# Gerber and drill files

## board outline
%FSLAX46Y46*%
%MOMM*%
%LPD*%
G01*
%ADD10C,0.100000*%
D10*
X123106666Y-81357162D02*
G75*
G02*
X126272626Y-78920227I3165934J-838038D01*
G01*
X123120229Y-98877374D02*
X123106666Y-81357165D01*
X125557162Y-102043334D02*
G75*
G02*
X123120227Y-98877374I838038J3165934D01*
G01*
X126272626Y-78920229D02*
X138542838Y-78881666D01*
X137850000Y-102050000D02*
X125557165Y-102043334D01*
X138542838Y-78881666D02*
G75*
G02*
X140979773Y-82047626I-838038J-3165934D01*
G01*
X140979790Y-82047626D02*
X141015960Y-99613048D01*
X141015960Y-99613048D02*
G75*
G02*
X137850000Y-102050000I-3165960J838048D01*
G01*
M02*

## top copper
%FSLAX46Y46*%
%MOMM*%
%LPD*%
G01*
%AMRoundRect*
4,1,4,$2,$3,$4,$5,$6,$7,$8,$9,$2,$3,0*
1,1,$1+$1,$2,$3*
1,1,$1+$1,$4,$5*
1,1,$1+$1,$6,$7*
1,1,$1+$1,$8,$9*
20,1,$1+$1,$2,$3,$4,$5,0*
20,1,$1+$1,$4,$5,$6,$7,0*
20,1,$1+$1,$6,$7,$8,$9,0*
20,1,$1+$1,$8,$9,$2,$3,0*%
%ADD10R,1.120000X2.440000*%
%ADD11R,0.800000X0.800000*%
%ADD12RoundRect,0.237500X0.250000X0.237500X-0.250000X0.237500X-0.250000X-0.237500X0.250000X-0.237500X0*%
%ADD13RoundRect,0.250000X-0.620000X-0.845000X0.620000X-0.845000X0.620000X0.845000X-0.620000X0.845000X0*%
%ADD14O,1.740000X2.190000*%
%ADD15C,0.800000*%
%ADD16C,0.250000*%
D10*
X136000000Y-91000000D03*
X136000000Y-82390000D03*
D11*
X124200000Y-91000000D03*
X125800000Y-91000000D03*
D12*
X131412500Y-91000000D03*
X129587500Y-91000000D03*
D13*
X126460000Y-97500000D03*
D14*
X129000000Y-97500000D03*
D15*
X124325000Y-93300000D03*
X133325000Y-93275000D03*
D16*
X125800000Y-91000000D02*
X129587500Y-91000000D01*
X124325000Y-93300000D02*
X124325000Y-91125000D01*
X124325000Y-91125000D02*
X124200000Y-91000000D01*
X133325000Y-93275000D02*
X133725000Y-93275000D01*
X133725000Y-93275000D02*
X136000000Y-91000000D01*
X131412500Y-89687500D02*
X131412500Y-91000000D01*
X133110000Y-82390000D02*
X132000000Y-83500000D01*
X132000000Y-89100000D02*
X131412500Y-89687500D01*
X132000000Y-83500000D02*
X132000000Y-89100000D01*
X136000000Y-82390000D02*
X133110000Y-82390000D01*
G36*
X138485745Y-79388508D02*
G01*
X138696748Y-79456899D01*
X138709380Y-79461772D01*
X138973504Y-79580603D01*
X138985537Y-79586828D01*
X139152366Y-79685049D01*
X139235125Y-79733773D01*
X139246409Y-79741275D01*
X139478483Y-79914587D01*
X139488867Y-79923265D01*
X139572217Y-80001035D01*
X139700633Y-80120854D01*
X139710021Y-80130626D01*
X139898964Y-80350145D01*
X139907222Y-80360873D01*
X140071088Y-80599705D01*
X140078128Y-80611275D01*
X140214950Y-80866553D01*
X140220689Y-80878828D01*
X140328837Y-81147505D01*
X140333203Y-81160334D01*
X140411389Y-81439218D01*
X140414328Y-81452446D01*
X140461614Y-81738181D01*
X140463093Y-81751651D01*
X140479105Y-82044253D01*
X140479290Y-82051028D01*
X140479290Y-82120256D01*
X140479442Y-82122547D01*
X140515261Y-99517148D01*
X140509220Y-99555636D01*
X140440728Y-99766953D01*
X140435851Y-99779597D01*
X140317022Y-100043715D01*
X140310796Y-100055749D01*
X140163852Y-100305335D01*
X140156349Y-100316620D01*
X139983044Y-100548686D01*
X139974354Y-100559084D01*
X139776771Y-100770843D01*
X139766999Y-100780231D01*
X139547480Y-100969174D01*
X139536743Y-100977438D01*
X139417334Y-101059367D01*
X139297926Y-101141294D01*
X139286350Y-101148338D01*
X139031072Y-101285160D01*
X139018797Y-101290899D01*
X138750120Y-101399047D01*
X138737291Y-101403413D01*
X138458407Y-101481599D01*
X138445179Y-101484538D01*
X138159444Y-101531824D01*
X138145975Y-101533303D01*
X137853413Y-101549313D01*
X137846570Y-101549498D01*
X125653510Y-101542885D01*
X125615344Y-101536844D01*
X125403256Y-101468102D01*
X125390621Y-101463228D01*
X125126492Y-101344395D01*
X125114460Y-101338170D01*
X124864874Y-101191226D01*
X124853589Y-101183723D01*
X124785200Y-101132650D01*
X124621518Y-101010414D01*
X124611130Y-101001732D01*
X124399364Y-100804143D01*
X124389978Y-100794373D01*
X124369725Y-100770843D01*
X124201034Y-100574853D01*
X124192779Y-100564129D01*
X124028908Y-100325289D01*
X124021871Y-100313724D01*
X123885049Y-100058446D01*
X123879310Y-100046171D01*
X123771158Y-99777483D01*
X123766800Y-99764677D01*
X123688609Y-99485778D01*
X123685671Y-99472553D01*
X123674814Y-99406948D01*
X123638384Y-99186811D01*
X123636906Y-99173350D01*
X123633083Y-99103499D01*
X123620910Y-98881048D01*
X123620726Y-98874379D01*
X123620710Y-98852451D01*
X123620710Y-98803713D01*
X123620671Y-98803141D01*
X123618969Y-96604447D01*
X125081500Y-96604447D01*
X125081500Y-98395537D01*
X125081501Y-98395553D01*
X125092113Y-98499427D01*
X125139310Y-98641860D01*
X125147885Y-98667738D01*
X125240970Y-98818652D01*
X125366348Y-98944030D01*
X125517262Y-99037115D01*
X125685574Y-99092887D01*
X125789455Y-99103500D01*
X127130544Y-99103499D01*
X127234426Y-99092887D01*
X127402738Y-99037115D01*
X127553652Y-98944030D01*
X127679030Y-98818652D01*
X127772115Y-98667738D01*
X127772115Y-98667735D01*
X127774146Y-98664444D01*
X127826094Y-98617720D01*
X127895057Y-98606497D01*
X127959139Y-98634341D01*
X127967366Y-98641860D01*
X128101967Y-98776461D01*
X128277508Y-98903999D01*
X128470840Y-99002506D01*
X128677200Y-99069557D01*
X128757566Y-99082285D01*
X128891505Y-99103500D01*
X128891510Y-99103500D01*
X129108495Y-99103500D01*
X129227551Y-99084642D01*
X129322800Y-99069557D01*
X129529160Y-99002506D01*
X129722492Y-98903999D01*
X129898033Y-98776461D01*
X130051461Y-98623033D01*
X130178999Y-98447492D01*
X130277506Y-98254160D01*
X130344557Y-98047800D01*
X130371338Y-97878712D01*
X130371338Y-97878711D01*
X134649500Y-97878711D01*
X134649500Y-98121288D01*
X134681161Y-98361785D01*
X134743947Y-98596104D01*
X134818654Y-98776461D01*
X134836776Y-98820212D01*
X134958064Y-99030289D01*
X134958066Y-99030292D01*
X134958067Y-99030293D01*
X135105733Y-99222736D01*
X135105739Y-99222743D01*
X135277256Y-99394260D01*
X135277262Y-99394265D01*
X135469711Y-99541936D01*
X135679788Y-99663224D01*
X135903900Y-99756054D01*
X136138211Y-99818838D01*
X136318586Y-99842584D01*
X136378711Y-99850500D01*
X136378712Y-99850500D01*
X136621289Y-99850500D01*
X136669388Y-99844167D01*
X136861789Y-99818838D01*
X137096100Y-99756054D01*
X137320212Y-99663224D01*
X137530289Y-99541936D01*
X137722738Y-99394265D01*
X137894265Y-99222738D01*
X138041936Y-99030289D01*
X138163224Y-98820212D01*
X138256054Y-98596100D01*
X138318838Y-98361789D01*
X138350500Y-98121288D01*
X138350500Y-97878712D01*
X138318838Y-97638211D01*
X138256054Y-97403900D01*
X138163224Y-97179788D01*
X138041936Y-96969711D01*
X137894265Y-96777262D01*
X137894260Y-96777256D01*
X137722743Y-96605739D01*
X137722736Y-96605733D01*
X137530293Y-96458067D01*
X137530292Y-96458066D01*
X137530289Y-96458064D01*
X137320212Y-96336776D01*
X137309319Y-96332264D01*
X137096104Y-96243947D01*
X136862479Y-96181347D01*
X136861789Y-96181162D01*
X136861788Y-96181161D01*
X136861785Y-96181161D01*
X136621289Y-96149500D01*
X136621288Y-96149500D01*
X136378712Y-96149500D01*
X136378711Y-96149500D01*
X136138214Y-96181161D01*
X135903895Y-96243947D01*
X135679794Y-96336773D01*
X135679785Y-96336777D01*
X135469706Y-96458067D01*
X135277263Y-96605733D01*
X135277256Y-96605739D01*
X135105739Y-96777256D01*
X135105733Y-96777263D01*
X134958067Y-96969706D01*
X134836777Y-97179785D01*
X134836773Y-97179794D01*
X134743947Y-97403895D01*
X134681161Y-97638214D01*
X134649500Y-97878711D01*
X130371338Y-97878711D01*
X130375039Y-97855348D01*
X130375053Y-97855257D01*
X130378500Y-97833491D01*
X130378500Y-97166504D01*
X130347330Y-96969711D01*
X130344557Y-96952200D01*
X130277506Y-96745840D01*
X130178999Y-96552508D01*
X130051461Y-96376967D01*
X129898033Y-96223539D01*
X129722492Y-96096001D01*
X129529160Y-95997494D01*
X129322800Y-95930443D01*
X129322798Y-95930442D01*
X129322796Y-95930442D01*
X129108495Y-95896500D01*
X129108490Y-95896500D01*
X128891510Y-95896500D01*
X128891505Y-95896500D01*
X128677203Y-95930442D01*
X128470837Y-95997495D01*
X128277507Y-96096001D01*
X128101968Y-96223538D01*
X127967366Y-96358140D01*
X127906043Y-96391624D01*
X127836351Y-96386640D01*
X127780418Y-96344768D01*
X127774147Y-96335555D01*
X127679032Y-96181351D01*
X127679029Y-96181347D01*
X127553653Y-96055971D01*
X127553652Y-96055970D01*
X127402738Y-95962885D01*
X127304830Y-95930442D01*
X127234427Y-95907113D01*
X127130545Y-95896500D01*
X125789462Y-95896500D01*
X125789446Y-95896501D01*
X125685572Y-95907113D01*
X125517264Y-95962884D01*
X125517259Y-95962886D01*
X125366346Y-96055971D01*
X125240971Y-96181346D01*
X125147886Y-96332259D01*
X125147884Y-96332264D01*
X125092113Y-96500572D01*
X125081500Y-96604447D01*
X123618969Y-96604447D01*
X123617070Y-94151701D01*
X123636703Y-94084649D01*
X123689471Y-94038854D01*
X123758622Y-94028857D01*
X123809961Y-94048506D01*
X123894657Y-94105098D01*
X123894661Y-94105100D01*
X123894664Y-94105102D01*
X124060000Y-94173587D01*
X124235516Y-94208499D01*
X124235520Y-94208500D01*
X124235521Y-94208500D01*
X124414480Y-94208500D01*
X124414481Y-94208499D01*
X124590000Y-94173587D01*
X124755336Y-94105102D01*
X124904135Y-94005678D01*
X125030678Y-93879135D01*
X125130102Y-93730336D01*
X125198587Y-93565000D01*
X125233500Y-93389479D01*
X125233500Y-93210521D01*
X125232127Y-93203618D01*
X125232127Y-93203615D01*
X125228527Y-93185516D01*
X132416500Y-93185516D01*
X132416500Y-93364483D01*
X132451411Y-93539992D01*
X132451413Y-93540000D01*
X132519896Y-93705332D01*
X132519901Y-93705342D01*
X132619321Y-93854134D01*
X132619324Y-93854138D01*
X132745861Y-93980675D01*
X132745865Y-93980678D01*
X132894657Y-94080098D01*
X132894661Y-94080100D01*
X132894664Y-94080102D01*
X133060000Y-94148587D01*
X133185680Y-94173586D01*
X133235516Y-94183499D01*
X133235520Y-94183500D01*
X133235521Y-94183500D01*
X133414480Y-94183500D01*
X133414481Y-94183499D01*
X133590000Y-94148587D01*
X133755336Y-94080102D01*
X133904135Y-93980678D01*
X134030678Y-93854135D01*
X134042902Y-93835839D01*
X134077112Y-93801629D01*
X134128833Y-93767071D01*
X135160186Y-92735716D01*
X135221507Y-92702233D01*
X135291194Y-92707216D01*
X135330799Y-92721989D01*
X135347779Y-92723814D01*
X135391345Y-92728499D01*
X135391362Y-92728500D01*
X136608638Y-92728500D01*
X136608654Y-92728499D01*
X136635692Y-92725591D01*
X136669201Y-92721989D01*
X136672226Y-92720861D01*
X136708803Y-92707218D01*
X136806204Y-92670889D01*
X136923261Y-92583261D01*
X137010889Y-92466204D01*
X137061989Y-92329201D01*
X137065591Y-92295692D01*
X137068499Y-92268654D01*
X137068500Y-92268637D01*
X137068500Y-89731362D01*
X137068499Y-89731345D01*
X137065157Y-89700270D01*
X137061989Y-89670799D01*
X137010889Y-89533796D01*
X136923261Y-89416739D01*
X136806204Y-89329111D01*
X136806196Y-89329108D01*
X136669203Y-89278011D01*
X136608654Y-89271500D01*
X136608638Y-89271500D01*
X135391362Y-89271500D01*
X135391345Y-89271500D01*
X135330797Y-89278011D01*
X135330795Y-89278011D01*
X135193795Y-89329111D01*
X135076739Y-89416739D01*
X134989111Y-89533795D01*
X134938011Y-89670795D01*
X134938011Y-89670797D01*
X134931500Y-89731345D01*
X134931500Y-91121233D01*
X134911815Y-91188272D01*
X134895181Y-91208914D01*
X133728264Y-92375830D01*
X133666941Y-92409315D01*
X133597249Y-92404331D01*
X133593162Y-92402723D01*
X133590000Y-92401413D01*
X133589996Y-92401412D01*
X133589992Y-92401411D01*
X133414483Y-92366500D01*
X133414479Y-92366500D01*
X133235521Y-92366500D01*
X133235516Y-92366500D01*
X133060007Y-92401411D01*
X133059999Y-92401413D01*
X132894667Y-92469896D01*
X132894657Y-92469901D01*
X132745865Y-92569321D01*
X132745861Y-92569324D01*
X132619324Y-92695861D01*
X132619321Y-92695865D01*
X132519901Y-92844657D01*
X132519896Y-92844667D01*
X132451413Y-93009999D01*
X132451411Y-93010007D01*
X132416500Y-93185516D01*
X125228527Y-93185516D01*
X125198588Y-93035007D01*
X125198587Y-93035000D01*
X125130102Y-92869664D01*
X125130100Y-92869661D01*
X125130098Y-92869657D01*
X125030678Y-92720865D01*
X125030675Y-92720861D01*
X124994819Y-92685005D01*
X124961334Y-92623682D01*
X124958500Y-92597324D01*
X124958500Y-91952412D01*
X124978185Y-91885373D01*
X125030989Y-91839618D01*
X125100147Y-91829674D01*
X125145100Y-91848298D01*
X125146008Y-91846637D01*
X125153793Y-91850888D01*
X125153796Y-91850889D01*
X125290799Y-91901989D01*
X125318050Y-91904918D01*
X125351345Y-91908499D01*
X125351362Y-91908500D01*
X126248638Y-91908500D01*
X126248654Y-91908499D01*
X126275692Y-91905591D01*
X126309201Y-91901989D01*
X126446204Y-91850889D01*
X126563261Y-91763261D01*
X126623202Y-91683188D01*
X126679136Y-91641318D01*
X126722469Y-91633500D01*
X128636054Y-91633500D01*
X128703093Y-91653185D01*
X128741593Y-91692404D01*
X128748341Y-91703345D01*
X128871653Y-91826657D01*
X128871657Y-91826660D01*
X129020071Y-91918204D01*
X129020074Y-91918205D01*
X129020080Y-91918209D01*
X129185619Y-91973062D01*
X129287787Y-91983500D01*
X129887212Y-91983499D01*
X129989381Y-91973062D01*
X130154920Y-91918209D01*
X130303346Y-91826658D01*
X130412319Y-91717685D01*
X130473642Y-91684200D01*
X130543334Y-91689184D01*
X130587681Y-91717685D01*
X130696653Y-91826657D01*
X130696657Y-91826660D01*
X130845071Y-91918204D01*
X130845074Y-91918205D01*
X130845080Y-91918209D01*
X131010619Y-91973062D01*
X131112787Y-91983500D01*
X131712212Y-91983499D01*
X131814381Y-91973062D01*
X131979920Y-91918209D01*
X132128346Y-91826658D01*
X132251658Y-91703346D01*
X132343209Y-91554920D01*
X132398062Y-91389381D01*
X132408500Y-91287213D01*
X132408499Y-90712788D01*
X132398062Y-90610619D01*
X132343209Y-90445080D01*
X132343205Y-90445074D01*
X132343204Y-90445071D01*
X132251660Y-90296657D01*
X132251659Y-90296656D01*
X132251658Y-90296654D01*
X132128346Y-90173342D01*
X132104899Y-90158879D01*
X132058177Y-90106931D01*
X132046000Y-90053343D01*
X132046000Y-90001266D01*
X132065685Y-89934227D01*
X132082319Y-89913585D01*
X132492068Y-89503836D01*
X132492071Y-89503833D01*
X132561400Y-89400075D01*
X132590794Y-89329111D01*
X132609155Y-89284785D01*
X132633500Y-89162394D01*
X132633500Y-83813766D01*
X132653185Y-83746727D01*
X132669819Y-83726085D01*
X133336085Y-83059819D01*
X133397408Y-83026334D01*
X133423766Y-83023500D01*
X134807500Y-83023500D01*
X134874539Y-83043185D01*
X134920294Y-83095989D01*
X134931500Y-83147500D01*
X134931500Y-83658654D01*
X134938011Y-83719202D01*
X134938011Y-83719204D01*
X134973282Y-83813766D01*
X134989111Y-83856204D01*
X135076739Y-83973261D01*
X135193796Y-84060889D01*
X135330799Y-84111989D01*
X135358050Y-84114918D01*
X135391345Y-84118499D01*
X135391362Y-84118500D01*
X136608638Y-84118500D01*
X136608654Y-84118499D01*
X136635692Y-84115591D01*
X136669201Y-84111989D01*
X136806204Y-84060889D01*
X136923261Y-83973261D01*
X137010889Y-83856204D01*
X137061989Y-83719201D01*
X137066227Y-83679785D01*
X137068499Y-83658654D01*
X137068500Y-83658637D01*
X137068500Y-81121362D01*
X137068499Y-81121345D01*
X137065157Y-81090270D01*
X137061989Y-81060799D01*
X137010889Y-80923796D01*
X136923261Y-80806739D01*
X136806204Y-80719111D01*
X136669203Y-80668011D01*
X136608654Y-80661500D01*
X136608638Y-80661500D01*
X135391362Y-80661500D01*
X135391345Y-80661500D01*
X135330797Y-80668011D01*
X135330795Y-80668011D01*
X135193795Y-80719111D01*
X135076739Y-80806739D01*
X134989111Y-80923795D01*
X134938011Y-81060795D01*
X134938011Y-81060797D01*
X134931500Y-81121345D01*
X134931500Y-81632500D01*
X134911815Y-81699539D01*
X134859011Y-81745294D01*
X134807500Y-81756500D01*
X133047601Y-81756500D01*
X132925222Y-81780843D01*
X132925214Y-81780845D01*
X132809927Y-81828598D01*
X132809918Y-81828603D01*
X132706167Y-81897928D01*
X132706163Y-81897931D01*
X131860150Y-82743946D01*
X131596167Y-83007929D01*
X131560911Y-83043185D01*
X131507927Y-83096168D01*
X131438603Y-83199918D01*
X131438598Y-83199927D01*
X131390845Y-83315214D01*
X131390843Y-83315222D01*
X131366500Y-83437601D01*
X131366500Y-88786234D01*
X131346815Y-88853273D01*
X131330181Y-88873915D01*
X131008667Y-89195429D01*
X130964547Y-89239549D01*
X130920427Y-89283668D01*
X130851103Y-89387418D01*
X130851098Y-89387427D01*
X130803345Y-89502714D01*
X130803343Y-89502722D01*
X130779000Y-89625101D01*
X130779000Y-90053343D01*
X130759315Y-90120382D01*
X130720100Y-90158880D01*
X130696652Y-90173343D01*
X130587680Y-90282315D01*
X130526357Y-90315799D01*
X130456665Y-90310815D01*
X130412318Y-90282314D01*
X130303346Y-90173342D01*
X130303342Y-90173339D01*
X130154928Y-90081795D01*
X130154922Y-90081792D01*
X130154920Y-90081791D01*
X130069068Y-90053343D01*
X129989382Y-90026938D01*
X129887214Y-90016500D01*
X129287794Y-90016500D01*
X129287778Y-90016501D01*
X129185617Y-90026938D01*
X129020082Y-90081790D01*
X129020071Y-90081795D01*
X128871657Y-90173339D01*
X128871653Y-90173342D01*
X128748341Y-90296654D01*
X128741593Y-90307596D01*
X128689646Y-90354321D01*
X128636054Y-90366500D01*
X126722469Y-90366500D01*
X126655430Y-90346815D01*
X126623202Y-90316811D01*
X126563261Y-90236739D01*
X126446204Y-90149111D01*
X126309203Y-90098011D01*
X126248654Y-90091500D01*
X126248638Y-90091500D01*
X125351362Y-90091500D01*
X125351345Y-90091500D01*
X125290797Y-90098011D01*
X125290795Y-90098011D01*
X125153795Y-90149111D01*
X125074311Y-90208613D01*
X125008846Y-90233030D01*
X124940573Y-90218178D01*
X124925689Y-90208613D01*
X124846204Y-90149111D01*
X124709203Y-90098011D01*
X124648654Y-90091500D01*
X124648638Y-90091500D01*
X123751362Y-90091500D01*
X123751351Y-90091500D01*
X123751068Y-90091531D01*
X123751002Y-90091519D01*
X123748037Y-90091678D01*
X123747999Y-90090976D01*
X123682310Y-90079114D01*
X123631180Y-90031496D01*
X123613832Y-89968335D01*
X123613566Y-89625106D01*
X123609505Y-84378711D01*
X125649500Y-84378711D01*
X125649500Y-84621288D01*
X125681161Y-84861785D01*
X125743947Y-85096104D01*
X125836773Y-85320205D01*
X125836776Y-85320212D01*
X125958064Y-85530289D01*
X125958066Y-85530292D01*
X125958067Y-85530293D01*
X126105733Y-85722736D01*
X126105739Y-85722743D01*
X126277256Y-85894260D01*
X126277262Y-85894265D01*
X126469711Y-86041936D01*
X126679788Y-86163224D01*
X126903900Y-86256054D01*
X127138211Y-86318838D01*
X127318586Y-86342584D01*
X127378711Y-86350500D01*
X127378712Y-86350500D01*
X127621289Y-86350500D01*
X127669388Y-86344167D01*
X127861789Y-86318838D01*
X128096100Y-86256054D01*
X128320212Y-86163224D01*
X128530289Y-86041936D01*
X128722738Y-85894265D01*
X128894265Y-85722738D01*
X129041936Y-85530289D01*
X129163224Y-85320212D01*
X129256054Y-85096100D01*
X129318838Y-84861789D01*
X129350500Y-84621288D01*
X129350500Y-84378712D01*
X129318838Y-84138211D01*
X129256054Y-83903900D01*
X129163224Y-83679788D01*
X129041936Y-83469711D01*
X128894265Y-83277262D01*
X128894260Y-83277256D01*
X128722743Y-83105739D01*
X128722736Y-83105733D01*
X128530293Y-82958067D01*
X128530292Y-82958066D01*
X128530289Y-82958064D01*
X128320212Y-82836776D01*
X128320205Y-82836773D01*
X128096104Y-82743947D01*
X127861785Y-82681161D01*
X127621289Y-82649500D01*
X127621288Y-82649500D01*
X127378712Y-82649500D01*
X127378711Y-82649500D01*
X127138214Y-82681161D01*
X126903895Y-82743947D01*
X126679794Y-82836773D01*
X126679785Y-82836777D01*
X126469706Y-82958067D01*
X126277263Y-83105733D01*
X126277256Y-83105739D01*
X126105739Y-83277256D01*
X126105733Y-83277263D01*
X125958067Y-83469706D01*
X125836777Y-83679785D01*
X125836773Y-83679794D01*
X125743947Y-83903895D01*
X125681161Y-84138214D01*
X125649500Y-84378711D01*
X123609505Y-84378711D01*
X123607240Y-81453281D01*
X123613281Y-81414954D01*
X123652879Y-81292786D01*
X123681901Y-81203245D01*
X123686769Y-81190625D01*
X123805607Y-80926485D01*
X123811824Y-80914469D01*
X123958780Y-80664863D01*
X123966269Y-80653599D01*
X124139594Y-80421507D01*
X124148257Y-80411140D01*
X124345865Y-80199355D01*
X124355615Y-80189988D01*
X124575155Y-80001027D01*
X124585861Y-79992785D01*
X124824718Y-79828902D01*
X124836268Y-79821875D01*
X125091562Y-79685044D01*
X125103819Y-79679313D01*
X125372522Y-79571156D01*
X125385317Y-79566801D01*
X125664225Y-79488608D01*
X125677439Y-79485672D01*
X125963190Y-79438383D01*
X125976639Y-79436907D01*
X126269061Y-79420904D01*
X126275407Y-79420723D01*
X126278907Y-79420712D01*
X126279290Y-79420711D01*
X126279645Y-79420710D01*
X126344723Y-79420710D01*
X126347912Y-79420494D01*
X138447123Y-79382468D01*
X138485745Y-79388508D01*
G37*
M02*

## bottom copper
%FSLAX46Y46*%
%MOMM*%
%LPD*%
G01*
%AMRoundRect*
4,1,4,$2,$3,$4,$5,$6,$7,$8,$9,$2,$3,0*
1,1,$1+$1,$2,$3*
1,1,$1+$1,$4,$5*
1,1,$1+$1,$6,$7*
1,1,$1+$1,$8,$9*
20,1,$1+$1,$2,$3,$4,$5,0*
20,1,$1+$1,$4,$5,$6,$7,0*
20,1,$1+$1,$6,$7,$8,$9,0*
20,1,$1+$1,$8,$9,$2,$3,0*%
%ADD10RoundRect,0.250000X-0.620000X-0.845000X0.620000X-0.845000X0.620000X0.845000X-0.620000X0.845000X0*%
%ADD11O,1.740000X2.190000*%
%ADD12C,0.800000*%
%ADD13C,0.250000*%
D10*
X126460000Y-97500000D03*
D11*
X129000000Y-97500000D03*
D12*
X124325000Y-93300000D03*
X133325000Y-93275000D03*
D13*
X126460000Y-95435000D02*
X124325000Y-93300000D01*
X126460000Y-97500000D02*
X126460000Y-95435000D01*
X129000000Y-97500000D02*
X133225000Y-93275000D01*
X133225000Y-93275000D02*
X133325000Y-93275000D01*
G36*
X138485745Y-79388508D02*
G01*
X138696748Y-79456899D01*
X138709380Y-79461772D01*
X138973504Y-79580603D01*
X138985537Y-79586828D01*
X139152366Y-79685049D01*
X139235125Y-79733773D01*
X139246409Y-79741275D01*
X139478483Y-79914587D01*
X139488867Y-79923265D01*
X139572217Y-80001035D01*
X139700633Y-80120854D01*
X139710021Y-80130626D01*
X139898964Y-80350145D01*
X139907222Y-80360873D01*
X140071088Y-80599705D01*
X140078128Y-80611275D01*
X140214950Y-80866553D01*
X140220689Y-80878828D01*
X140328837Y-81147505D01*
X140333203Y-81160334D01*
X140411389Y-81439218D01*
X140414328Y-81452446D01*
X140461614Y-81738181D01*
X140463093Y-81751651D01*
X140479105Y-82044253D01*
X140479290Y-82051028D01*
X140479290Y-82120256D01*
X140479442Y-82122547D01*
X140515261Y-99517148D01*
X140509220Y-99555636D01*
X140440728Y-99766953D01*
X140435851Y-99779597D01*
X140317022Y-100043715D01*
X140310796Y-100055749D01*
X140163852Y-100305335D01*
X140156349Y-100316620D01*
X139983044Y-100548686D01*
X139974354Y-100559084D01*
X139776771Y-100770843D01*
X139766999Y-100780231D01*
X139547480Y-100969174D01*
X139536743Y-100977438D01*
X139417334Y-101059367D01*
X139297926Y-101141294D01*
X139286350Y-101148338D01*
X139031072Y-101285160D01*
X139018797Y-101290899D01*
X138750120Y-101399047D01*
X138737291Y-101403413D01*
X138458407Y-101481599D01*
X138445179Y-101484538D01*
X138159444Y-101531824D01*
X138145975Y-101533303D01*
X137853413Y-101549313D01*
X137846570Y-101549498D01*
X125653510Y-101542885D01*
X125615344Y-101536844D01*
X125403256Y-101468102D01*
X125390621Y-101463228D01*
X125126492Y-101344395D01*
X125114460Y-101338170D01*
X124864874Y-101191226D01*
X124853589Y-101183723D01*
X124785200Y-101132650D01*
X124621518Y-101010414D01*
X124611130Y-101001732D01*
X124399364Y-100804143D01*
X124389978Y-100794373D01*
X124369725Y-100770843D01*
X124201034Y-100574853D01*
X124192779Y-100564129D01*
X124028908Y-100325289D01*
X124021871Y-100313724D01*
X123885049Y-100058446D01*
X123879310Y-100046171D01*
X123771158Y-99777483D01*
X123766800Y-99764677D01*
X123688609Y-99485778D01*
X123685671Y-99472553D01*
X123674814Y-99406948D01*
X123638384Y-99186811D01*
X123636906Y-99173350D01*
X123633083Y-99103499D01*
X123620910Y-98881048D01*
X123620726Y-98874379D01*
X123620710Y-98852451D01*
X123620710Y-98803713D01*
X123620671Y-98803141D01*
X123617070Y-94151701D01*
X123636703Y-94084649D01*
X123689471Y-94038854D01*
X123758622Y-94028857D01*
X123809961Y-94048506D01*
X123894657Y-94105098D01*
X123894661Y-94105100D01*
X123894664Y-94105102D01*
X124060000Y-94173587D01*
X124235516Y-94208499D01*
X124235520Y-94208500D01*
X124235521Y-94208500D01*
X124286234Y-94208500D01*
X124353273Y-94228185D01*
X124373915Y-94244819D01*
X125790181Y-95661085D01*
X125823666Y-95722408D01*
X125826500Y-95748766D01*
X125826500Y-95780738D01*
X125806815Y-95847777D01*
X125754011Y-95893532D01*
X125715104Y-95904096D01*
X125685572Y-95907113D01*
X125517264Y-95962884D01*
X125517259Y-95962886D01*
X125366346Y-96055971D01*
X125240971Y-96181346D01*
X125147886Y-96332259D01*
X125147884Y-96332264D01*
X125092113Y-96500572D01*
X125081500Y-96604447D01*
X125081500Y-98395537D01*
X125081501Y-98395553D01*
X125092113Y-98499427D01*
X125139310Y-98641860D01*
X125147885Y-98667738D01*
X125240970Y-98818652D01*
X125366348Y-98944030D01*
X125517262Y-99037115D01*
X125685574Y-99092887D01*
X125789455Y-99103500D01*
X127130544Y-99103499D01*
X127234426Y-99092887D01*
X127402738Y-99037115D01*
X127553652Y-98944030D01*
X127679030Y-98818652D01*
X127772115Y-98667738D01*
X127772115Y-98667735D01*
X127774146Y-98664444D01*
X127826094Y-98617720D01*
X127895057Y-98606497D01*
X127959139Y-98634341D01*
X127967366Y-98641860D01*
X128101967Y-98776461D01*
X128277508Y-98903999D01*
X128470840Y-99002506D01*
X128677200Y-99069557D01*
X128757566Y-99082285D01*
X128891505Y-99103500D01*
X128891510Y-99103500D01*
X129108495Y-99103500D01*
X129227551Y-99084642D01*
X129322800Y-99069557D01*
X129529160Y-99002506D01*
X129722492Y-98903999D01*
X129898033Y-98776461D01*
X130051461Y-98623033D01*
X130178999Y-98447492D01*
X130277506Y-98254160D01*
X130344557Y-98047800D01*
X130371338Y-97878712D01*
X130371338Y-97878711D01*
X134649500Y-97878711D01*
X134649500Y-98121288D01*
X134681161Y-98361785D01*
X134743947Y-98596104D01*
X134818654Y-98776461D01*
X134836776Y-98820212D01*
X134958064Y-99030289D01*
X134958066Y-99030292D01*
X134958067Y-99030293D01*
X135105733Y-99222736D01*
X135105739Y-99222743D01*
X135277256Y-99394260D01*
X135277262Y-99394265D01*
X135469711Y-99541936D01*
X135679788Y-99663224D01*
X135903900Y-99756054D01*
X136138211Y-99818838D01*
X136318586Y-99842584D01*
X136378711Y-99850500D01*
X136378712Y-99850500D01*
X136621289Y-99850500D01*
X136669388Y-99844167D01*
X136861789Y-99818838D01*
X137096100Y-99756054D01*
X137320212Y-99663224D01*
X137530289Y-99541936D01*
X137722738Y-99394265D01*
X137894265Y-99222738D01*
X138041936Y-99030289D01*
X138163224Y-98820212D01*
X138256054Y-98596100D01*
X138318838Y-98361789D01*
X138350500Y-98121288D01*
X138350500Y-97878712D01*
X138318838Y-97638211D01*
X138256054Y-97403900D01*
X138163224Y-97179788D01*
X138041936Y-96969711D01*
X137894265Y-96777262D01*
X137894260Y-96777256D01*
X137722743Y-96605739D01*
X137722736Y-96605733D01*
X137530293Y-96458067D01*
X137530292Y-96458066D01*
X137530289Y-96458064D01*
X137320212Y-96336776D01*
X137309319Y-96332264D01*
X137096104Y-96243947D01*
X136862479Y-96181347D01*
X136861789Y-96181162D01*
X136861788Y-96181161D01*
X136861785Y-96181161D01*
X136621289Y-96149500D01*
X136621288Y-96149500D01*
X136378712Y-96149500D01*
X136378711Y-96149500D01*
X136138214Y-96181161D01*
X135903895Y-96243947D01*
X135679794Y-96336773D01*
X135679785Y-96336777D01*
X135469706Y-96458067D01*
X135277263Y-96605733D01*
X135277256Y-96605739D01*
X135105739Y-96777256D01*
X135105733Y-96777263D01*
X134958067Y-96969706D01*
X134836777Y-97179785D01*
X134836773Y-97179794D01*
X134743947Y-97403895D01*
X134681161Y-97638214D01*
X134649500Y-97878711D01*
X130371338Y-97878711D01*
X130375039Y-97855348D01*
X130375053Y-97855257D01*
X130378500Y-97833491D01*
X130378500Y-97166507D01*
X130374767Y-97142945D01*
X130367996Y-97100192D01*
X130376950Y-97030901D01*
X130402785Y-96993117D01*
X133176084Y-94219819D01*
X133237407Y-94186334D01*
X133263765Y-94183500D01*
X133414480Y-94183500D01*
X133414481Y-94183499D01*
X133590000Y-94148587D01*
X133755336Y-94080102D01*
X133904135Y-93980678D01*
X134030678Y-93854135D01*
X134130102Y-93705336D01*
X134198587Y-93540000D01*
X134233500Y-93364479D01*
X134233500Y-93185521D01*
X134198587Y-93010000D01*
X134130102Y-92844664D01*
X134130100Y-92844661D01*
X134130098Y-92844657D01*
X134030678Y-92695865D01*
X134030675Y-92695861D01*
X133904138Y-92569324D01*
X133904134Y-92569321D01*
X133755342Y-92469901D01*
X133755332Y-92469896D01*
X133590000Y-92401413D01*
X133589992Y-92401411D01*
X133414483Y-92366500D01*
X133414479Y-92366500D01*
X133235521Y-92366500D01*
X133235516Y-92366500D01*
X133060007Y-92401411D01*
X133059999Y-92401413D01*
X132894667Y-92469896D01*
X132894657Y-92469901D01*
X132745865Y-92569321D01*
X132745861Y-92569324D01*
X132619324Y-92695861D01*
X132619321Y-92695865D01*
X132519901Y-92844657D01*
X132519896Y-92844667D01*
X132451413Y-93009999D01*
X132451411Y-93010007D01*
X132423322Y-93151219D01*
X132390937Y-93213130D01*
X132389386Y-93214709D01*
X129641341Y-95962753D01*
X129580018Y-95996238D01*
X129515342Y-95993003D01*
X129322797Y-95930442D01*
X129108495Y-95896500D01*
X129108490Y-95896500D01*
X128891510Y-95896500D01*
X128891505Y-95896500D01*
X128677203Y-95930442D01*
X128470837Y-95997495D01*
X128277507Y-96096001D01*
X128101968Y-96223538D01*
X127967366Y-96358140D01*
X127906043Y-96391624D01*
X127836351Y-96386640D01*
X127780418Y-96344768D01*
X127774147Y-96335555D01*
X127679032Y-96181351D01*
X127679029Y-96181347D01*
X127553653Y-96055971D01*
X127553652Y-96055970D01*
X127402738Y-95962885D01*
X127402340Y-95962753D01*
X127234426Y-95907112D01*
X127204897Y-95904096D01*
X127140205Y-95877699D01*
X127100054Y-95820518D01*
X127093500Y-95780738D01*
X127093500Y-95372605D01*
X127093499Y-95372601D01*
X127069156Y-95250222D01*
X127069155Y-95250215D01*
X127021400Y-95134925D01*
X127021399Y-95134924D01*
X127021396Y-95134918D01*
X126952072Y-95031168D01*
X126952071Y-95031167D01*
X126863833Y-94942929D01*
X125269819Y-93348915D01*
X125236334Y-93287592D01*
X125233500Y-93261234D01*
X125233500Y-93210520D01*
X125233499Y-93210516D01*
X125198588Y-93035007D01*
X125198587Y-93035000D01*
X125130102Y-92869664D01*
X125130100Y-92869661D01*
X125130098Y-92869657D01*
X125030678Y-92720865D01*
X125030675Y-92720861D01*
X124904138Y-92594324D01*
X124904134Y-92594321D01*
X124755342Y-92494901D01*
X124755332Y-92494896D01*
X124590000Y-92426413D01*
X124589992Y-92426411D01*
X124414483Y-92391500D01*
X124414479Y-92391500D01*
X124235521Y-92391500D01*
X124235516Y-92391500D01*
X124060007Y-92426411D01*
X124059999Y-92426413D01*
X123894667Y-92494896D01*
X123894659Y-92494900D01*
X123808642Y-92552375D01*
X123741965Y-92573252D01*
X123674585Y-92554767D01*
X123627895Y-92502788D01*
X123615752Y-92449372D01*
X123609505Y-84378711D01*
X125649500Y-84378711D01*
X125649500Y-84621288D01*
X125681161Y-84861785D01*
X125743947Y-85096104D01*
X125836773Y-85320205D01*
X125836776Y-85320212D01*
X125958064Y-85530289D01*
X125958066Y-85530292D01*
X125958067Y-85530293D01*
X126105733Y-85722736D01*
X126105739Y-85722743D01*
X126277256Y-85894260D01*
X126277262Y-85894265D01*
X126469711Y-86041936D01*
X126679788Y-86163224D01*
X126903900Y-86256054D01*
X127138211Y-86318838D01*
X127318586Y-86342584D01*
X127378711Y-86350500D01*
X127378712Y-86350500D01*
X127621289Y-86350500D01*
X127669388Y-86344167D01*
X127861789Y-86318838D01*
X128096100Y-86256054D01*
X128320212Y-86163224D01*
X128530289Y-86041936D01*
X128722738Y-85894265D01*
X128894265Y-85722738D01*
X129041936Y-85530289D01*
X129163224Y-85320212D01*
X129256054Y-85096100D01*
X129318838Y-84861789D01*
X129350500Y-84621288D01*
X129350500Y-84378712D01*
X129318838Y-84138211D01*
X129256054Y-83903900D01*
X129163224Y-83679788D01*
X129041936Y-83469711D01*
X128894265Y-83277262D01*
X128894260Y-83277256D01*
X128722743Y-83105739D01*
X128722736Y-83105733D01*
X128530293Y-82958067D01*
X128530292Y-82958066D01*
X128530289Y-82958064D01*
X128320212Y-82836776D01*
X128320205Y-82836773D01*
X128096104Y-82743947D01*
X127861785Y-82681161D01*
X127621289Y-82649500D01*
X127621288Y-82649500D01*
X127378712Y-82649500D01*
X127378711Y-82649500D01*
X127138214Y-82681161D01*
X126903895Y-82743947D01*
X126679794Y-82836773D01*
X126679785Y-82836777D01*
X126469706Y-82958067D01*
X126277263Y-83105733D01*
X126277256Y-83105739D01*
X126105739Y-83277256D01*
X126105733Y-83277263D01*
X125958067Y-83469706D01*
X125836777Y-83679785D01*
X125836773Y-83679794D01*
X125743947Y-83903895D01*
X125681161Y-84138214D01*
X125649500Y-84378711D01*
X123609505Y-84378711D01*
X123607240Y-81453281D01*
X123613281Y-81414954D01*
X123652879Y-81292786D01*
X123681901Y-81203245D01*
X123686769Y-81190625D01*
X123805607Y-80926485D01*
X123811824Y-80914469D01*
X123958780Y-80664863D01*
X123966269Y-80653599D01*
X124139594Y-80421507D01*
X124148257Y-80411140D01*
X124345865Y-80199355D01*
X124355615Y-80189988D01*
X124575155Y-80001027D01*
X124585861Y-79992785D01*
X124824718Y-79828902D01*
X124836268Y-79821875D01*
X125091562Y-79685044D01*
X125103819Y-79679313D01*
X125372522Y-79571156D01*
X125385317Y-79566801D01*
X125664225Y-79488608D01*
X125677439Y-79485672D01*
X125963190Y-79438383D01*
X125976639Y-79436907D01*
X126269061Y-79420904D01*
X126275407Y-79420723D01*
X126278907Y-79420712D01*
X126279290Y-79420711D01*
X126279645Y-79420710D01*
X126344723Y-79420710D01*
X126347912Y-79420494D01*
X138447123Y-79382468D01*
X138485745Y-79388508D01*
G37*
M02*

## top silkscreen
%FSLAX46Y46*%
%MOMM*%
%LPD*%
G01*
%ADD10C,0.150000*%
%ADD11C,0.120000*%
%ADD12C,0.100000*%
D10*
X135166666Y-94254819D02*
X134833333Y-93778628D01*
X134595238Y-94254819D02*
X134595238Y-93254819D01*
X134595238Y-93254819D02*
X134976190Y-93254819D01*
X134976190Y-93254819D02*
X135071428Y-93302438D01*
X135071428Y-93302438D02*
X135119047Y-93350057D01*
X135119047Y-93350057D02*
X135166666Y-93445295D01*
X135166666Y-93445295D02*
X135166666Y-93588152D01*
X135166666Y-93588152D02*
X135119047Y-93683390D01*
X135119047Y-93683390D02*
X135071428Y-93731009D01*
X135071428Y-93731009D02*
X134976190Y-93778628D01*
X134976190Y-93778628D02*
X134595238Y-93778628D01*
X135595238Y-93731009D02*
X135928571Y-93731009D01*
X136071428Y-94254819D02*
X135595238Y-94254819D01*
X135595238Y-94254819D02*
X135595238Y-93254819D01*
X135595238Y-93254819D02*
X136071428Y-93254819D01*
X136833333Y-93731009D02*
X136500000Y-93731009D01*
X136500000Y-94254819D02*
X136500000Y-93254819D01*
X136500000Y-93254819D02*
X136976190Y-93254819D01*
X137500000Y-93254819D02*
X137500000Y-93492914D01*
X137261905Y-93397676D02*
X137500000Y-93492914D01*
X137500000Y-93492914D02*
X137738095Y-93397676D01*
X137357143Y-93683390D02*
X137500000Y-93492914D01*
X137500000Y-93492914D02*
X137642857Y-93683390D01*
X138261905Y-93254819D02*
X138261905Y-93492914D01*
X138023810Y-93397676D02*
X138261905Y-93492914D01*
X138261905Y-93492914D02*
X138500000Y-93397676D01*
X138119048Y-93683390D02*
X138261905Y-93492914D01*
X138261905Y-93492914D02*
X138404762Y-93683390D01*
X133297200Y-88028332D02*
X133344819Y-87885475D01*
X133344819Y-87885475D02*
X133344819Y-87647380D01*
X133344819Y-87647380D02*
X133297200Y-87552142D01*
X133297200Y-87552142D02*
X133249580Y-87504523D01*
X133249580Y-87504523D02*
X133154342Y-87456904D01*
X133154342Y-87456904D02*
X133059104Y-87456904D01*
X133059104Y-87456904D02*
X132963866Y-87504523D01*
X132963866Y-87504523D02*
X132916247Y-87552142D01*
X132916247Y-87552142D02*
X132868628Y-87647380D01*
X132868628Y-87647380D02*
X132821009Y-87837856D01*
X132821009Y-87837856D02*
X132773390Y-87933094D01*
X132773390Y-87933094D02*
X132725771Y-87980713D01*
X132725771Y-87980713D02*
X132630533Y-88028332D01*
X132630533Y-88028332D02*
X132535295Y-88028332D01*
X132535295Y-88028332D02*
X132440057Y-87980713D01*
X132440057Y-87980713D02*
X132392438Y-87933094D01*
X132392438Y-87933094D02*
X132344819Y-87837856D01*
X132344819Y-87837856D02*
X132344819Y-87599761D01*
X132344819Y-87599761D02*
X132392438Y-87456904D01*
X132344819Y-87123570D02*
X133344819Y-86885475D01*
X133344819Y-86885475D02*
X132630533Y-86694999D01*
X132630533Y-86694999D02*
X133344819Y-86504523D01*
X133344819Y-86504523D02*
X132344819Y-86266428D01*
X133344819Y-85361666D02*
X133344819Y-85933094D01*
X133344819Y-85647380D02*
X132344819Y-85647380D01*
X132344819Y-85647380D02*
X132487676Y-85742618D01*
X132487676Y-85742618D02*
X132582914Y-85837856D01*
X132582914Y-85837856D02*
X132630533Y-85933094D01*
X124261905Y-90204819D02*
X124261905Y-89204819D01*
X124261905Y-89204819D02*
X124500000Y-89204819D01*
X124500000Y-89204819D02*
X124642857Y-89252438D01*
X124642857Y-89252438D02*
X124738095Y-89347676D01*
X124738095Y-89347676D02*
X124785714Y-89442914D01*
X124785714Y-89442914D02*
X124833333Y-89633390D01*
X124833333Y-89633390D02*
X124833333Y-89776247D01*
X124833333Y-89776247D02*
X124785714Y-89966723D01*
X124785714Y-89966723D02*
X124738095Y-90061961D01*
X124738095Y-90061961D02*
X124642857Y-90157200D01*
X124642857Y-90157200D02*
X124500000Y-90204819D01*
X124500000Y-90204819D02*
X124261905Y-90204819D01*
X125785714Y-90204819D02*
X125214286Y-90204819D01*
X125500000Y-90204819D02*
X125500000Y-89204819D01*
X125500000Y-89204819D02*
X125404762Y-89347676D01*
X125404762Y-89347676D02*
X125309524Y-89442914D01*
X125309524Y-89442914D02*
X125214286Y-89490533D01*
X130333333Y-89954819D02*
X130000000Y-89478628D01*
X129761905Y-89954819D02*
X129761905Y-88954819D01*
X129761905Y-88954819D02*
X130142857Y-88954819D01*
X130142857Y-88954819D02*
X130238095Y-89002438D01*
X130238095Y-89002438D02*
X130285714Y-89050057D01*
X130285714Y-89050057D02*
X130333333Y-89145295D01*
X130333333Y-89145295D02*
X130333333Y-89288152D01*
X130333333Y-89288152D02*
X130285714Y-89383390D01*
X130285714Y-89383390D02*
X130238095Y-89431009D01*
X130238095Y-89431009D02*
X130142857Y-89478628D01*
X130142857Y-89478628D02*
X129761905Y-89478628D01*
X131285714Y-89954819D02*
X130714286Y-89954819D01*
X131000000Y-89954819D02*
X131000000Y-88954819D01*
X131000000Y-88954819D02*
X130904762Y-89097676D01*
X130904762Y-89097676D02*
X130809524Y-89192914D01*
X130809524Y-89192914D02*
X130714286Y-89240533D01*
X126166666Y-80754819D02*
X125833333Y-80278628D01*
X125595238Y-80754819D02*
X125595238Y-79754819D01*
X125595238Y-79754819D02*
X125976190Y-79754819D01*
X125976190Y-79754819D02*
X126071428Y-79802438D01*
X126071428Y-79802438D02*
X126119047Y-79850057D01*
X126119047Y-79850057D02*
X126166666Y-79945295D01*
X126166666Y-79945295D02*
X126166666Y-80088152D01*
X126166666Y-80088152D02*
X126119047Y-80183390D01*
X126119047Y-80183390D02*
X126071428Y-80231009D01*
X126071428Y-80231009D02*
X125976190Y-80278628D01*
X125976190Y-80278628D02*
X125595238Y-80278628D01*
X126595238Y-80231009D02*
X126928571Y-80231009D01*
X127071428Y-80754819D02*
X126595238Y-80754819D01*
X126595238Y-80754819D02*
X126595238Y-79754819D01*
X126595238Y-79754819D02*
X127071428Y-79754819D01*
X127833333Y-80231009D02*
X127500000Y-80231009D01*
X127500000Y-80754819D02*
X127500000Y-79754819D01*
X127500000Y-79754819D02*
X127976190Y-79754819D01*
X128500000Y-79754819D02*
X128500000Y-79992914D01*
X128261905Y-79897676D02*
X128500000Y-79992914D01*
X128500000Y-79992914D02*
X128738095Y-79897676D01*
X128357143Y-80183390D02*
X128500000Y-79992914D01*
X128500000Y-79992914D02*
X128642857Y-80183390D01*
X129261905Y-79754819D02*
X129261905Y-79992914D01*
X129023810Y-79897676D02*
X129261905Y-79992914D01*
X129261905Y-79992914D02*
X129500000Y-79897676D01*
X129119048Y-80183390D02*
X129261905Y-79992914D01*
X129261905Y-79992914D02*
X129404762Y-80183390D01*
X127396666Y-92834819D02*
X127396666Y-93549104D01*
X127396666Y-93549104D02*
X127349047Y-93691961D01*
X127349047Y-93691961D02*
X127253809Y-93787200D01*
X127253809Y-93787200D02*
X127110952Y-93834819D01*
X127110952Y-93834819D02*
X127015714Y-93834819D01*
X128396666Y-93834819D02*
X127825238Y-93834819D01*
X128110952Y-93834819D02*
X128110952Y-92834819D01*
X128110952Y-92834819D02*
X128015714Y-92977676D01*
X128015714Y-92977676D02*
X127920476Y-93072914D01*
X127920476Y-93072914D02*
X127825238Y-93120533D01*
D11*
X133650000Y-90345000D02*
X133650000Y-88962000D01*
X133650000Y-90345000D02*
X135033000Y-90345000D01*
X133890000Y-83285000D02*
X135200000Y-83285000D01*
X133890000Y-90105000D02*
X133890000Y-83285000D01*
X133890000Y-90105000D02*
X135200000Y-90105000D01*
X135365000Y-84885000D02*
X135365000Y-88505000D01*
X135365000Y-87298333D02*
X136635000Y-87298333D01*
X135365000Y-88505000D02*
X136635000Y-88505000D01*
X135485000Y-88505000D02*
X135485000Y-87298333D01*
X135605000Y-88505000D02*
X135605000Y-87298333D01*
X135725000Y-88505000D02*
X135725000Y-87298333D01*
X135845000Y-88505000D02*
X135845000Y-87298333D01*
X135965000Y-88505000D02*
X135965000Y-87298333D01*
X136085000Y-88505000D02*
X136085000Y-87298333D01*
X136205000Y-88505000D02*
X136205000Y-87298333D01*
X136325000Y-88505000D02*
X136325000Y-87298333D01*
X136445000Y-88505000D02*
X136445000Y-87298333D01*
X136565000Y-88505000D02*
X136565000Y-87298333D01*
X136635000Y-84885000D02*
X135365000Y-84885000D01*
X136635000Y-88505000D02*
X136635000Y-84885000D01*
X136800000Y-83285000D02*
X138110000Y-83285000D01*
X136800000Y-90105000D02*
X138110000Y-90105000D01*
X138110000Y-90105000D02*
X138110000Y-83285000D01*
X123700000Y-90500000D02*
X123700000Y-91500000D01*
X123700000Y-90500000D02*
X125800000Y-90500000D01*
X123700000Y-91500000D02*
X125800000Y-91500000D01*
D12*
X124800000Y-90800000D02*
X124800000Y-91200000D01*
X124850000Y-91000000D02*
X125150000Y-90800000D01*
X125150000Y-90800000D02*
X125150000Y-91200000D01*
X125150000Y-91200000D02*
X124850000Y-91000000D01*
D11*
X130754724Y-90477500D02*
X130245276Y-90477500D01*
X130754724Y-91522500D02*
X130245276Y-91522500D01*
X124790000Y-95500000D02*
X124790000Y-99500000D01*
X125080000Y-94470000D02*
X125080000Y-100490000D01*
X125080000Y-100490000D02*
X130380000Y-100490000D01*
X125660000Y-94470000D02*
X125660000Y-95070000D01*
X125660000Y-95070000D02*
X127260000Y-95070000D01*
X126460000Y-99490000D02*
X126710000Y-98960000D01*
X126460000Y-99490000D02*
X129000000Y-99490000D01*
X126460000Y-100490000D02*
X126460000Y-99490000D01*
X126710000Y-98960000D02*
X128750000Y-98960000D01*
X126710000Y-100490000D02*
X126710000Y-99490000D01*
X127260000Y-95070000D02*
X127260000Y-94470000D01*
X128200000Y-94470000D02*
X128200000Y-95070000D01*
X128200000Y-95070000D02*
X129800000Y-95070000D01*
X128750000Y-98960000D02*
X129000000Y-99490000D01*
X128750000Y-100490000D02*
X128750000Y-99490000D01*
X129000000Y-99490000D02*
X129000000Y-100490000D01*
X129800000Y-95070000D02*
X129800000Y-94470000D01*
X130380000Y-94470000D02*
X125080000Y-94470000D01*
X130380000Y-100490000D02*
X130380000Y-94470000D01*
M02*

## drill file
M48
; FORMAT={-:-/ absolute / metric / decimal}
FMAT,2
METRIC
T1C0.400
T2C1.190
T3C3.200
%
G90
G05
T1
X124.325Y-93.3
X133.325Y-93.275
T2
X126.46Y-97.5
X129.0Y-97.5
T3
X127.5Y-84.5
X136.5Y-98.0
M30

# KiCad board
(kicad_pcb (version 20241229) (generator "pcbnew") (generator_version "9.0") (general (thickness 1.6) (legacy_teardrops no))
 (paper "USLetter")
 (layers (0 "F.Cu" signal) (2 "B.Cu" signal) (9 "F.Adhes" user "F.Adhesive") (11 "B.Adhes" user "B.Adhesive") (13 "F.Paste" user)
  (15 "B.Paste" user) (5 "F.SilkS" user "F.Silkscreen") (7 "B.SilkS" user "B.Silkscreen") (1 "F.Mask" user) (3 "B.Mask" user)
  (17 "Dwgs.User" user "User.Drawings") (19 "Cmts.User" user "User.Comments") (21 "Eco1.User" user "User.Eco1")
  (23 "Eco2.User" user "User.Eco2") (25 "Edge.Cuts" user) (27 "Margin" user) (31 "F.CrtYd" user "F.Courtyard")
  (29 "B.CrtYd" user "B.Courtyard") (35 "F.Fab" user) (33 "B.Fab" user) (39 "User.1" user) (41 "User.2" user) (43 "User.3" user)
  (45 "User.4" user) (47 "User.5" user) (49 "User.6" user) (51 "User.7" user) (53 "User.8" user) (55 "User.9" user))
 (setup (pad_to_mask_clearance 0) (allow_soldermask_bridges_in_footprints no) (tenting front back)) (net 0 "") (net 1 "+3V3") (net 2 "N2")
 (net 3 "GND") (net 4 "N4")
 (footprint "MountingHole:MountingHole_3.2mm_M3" (layer "F.Cu") (at 136.5 98)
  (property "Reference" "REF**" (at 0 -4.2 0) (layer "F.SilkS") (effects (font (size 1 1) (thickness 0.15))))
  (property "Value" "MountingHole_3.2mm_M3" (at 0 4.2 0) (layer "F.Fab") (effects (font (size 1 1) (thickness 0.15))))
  (pad "" np_thru_hole circle (at 0 0) (size 3.2 3.2) (drill 3.2) (layers "*.Cu" "*.Mask")))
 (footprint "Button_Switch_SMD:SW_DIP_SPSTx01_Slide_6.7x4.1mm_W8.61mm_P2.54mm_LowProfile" (layer "F.Cu") (at 136 86.695 90)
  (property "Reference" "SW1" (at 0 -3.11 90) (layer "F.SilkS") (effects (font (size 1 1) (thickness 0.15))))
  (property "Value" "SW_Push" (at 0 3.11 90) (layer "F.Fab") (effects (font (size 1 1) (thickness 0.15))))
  (fp_line (start -3.65 -2.35) (end -2.267 -2.35) (stroke (width 0.12) (type solid)) (layer "F.SilkS"))
  (fp_line (start -3.65 -2.35) (end -3.65 -0.967) (stroke (width 0.12) (type solid)) (layer "F.SilkS"))
  (fp_line (start 3.41 -2.11) (end 3.41 -0.8) (stroke (width 0.12) (type solid)) (layer "F.SilkS"))
  (fp_line (start -3.41 -2.11) (end 3.41 -2.11) (stroke (width 0.12) (type solid)) (layer "F.SilkS"))
  (fp_line (start -3.41 -2.11) (end -3.41 -0.8) (stroke (width 0.12) (type solid)) (layer "F.SilkS"))
  (fp_line (start 1.81 -0.635) (end -1.81 -0.635) (stroke (width 0.12) (type solid)) (layer "F.SilkS"))
  (fp_line (start -0.603333 -0.635) (end -0.603333 0.635) (stroke (width 0.12) (type solid)) (layer "F.SilkS"))
  (fp_line (start -1.81 -0.635) (end -1.81 0.635) (stroke (width 0.12) (type solid)) (layer "F.SilkS"))
  (fp_line (start -1.81 -0.515) (end -0.603333 -0.515) (stroke (width 0.12) (type solid)) (layer "F.SilkS"))
  (fp_line (start -1.81 -0.395) (end -0.603333 -0.395) (stroke (width 0.12) (type solid)) (layer "F.SilkS"))
  (fp_line (start -1.81 -0.275) (end -0.603333 -0.275) (stroke (width 0.12) (type solid)) (layer "F.SilkS"))
  (fp_line (start -1.81 -0.155) (end -0.603333 -0.155) (stroke (width 0.12) (type solid)) (layer "F.SilkS"))
  (fp_line (start -1.81 -0.035) (end -0.603333 -0.035) (stroke (width 0.12) (type solid)) (layer "F.SilkS"))
  (fp_line (start -1.81 0.085) (end -0.603333 0.085) (stroke (width 0.12) (type solid)) (layer "F.SilkS"))
  (fp_line (start -1.81 0.205) (end -0.603333 0.205) (stroke (width 0.12) (type solid)) (layer "F.SilkS"))
  (fp_line (start -1.81 0.325) (end -0.603333 0.325) (stroke (width 0.12) (type solid)) (layer "F.SilkS"))
  (fp_line (start -1.81 0.445) (end -0.603333 0.445) (stroke (width 0.12) (type solid)) (layer "F.SilkS"))
  (fp_line (start -1.81 0.565) (end -0.603333 0.565) (stroke (width 0.12) (type solid)) (layer "F.SilkS"))
  (fp_line (start 1.81 0.635) (end 1.81 -0.635) (stroke (width 0.12) (type solid)) (layer "F.SilkS"))
  (fp_line (start -1.81 0.635) (end 1.81 0.635) (stroke (width 0.12) (type solid)) (layer "F.SilkS"))
  (fp_line (start 3.41 0.8) (end 3.41 2.11) (stroke (width 0.12) (type solid)) (layer "F.SilkS"))
  (fp_line (start -3.41 0.8) (end -3.41 2.11) (stroke (width 0.12) (type solid)) (layer "F.SilkS"))
  (fp_line (start -3.41 2.11) (end 3.41 2.11) (stroke (width 0.12) (type solid)) (layer "F.SilkS"))
  (pad "1" smd rect (at -4.305 0 90) (size 2.44 1.12) (layers "F.Cu" "F.Mask" "F.Paste") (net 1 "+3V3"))
  (pad "2" smd rect (at 4.305 0 90) (size 2.44 1.12) (layers "F.Cu" "F.Mask" "F.Paste") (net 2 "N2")))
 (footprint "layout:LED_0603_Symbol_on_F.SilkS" (layer "F.Cu") (at 125 91)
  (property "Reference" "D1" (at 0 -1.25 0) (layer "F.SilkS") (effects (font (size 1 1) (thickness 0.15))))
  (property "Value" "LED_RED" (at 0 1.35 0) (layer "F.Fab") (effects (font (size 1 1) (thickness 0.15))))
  (fp_line (start -1.3 -0.5) (end -1.3 0.5) (stroke (width 0.12) (type solid)) (layer "F.SilkS"))
  (fp_line (start -1.3 -0.5) (end 0.8 -0.5) (stroke (width 0.12) (type solid)) (layer "F.SilkS"))
  (fp_line (start -1.3 0.5) (end 0.8 0.5) (stroke (width 0.12) (type solid)) (layer "F.SilkS"))
  (fp_line (start -0.2 -0.2) (end -0.2 0.2) (stroke (width 0.1) (type solid)) (layer "F.SilkS"))
  (fp_line (start -0.15 0) (end 0.15 -0.2) (stroke (width 0.1) (type solid)) (layer "F.SilkS"))
  (fp_line (start 0.15 -0.2) (end 0.15 0.2) (stroke (width 0.1) (type solid)) (layer "F.SilkS"))
  (fp_line (start 0.15 0.2) (end -0.15 0) (stroke (width 0.1) (type solid)) (layer "F.SilkS"))
  (pad "1" smd rect (at -0.8 0 180) (size 0.8 0.8) (layers "F.Cu" "F.Mask" "F.Paste") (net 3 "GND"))
  (pad "2" smd rect (at 0.8 0 180) (size 0.8 0.8) (layers "F.Cu" "F.Mask" "F.Paste") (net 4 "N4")))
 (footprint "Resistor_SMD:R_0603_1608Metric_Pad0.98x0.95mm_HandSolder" (layer "F.Cu") (at 130.5 91 180)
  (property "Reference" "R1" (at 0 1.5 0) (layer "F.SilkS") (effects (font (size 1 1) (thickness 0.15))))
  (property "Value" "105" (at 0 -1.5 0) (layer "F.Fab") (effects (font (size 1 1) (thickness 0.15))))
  (fp_line (start -0.254724 0.5225) (end 0.254724 0.5225) (stroke (width 0.12) (type solid)) (layer "F.SilkS"))
  (fp_line (start -0.254724 -0.5225) (end 0.254724 -0.5225) (stroke (width 0.12) (type solid)) (layer "F.SilkS"))
  (pad "1" smd roundrect (at -0.9125 0 180) (size 0.975 0.95) (layers "F.Cu" "F.Mask" "F.Paste") (roundrect_rratio 0.25) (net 2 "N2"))
  (pad "2" smd roundrect (at 0.9125 0 180) (size 0.975 0.95) (layers "F.Cu" "F.Mask" "F.Paste") (roundrect_rratio 0.25) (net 4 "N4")))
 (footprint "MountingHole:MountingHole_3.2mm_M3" (layer "F.Cu") (at 127.5 84.5)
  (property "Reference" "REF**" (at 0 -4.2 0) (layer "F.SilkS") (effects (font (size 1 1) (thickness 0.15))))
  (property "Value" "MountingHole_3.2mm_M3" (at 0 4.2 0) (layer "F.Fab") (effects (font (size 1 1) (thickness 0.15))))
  (pad "" np_thru_hole circle (at 0 0) (size 3.2 3.2) (drill 3.2) (layers "*.Cu" "*.Mask")))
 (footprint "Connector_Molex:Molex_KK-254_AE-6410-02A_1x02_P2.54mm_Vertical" (layer "F.Cu") (at 126.46 97.5)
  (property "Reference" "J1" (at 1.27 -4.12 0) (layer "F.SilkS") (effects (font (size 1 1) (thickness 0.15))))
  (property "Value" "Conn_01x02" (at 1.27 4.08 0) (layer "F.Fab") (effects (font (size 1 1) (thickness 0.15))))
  (fp_line (start -1.67 -2) (end -1.67 2) (stroke (width 0.12) (type solid)) (layer "F.SilkS"))
  (fp_line (start -1.38 -3.03) (end -1.38 2.99) (stroke (width 0.12) (type solid)) (layer "F.SilkS"))
  (fp_line (start -1.38 2.99) (end 3.92 2.99) (stroke (width 0.12) (type solid)) (layer "F.SilkS"))
  (fp_line (start -0.8 -3.03) (end -0.8 -2.43) (stroke (width 0.12) (type solid)) (layer "F.SilkS"))
  (fp_line (start -0.8 -2.43) (end 0.8 -2.43) (stroke (width 0.12) (type solid)) (layer "F.SilkS"))
  (fp_line (start 0 1.99) (end 0.25 1.46) (stroke (width 0.12) (type solid)) (layer "F.SilkS"))
  (fp_line (start 0 1.99) (end 2.54 1.99) (stroke (width 0.12) (type solid)) (layer "F.SilkS"))
  (fp_line (start 0 2.99) (end 0 1.99) (stroke (width 0.12) (type solid)) (layer "F.SilkS"))
  (fp_line (start 0.25 1.46) (end 2.29 1.46) (stroke (width 0.12) (type solid)) (layer "F.SilkS"))
  (fp_line (start 0.25 2.99) (end 0.25 1.99) (stroke (width 0.12) (type solid)) (layer "F.SilkS"))
  (fp_line (start 0.8 -2.43) (end 0.8 -3.03) (stroke (width 0.12) (type solid)) (layer "F.SilkS"))
  (fp_line (start 1.74 -3.03) (end 1.74 -2.43) (stroke (width 0.12) (type solid)) (layer "F.SilkS"))
  (fp_line (start 1.74 -2.43) (end 3.34 -2.43) (stroke (width 0.12) (type solid)) (layer "F.SilkS"))
  (fp_line (start 2.29 1.46) (end 2.54 1.99) (stroke (width 0.12) (type solid)) (layer "F.SilkS"))
  (fp_line (start 2.29 2.99) (end 2.29 1.99) (stroke (width 0.12) (type solid)) (layer "F.SilkS"))
  (fp_line (start 2.54 1.99) (end 2.54 2.99) (stroke (width 0.12) (type solid)) (layer "F.SilkS"))
  (fp_line (start 3.34 -2.43) (end 3.34 -3.03) (stroke (width 0.12) (type solid)) (layer "F.SilkS"))
  (fp_line (start 3.92 -3.03) (end -1.38 -3.03) (stroke (width 0.12) (type solid)) (layer "F.SilkS"))
  (fp_line (start 3.92 2.99) (end 3.92 -3.03) (stroke (width 0.12) (type solid)) (layer "F.SilkS"))
  (pad "1" thru_hole roundrect (at 0 0) (size 1.74 2.19) (drill 1.19) (layers "*.Cu" "*.Mask") (remove_unused_layers no)
   (roundrect_rratio 0.143678) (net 3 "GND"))
  (pad "2" thru_hole oval (at 2.54 0) (size 1.74 2.19) (drill 1.19) (layers "*.Cu" "*.Mask") (remove_unused_layers no) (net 1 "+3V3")))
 (gr_arc (start 123.106666 81.357162) (mid 124.275 79.6) (end 126.272626 78.92021) (stroke (width 0.1) (type default)) (layer "Edge.Cuts"))
 (gr_line (start 123.120229 98.877374) (end 123.106666 81.357165) (stroke (width 0.1) (type default)) (layer "Edge.Cuts"))
 (gr_arc (start 125.557162 102.043334) (mid 123.8 100.875) (end 123.12021 98.877374) (stroke (width 0.1) (type default)) (layer "Edge.Cuts"))
 (gr_line (start 126.272626 78.920229) (end 138.542838 78.881666) (stroke (width 0.1) (type default)) (layer "Edge.Cuts"))
 (gr_line (start 137.85 102.05) (end 125.557165 102.043334) (stroke (width 0.1) (type default)) (layer "Edge.Cuts"))
 (gr_arc (start 138.542838 78.881666) (mid 140.3 80.05) (end 140.97979 82.047626) (stroke (width 0.1) (type default)) (layer "Edge.Cuts"))
 (gr_line (start 140.97979 82.047626) (end 141.01596 99.613048) (stroke (width 0.1) (type default)) (layer "Edge.Cuts"))
 (gr_arc (start 141.01596 99.613048) (mid 139.847626 101.37021) (end 137.85 102.05) (stroke (width 0.1) (type default)) (layer "Edge.Cuts"))
 (segment (start 125.8 91) (end 129.5875 91) (width 0.25) (layer "F.Cu") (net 4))
 (segment (start 124.325 93.3) (end 124.325 91.125) (width 0.25) (layer "F.Cu") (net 3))
 (segment (start 124.325 91.125) (end 124.2 91) (width 0.25) (layer "F.Cu") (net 3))
 (via (at 124.325 93.3) (size 0.8) (drill 0.4) (layers "F.Cu" "B.Cu") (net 3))
 (segment (start 126.46 95.435) (end 124.325 93.3) (width 0.25) (layer "B.Cu") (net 3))
 (segment (start 126.46 97.5) (end 126.46 95.435) (width 0.25) (layer "B.Cu") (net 3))
 (segment (start 133.325 93.275) (end 133.725 93.275) (width 0.25) (layer "F.Cu") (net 1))
 (segment (start 133.725 93.275) (end 136 91) (width 0.25) (layer "F.Cu") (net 1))
 (via (at 133.325 93.275) (size 0.8) (drill 0.4) (layers "F.Cu" "B.Cu") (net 1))
 (segment (start 129 97.5) (end 133.225 93.275) (width 0.25) (layer "B.Cu") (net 1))
 (segment (start 133.225 93.275) (end 133.325 93.275) (width 0.25) (layer "B.Cu") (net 1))
 (segment (start 131.4125 89.6875) (end 131.4125 91) (width 0.25) (layer "F.Cu") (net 2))
 (segment (start 133.11 82.39) (end 132 83.5) (width 0.25) (layer "F.Cu") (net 2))
 (segment (start 132 89.1) (end 131.4125 89.6875) (width 0.25) (layer "F.Cu") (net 2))
 (segment (start 132 83.5) (end 132 89.1) (width 0.25) (layer "F.Cu") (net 2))
 (segment (start 136 82.39) (end 133.11 82.39) (width 0.25) (layer "F.Cu") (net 2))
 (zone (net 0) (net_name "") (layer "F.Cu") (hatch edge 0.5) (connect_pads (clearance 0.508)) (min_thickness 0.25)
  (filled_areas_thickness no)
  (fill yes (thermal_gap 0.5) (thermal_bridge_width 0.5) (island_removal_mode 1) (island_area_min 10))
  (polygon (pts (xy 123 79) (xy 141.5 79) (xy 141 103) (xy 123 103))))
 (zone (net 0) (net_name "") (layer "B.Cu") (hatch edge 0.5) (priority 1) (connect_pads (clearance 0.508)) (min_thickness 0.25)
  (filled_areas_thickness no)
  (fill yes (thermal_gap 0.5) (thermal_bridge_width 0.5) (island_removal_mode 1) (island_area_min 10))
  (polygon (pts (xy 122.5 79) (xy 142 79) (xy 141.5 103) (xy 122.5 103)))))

